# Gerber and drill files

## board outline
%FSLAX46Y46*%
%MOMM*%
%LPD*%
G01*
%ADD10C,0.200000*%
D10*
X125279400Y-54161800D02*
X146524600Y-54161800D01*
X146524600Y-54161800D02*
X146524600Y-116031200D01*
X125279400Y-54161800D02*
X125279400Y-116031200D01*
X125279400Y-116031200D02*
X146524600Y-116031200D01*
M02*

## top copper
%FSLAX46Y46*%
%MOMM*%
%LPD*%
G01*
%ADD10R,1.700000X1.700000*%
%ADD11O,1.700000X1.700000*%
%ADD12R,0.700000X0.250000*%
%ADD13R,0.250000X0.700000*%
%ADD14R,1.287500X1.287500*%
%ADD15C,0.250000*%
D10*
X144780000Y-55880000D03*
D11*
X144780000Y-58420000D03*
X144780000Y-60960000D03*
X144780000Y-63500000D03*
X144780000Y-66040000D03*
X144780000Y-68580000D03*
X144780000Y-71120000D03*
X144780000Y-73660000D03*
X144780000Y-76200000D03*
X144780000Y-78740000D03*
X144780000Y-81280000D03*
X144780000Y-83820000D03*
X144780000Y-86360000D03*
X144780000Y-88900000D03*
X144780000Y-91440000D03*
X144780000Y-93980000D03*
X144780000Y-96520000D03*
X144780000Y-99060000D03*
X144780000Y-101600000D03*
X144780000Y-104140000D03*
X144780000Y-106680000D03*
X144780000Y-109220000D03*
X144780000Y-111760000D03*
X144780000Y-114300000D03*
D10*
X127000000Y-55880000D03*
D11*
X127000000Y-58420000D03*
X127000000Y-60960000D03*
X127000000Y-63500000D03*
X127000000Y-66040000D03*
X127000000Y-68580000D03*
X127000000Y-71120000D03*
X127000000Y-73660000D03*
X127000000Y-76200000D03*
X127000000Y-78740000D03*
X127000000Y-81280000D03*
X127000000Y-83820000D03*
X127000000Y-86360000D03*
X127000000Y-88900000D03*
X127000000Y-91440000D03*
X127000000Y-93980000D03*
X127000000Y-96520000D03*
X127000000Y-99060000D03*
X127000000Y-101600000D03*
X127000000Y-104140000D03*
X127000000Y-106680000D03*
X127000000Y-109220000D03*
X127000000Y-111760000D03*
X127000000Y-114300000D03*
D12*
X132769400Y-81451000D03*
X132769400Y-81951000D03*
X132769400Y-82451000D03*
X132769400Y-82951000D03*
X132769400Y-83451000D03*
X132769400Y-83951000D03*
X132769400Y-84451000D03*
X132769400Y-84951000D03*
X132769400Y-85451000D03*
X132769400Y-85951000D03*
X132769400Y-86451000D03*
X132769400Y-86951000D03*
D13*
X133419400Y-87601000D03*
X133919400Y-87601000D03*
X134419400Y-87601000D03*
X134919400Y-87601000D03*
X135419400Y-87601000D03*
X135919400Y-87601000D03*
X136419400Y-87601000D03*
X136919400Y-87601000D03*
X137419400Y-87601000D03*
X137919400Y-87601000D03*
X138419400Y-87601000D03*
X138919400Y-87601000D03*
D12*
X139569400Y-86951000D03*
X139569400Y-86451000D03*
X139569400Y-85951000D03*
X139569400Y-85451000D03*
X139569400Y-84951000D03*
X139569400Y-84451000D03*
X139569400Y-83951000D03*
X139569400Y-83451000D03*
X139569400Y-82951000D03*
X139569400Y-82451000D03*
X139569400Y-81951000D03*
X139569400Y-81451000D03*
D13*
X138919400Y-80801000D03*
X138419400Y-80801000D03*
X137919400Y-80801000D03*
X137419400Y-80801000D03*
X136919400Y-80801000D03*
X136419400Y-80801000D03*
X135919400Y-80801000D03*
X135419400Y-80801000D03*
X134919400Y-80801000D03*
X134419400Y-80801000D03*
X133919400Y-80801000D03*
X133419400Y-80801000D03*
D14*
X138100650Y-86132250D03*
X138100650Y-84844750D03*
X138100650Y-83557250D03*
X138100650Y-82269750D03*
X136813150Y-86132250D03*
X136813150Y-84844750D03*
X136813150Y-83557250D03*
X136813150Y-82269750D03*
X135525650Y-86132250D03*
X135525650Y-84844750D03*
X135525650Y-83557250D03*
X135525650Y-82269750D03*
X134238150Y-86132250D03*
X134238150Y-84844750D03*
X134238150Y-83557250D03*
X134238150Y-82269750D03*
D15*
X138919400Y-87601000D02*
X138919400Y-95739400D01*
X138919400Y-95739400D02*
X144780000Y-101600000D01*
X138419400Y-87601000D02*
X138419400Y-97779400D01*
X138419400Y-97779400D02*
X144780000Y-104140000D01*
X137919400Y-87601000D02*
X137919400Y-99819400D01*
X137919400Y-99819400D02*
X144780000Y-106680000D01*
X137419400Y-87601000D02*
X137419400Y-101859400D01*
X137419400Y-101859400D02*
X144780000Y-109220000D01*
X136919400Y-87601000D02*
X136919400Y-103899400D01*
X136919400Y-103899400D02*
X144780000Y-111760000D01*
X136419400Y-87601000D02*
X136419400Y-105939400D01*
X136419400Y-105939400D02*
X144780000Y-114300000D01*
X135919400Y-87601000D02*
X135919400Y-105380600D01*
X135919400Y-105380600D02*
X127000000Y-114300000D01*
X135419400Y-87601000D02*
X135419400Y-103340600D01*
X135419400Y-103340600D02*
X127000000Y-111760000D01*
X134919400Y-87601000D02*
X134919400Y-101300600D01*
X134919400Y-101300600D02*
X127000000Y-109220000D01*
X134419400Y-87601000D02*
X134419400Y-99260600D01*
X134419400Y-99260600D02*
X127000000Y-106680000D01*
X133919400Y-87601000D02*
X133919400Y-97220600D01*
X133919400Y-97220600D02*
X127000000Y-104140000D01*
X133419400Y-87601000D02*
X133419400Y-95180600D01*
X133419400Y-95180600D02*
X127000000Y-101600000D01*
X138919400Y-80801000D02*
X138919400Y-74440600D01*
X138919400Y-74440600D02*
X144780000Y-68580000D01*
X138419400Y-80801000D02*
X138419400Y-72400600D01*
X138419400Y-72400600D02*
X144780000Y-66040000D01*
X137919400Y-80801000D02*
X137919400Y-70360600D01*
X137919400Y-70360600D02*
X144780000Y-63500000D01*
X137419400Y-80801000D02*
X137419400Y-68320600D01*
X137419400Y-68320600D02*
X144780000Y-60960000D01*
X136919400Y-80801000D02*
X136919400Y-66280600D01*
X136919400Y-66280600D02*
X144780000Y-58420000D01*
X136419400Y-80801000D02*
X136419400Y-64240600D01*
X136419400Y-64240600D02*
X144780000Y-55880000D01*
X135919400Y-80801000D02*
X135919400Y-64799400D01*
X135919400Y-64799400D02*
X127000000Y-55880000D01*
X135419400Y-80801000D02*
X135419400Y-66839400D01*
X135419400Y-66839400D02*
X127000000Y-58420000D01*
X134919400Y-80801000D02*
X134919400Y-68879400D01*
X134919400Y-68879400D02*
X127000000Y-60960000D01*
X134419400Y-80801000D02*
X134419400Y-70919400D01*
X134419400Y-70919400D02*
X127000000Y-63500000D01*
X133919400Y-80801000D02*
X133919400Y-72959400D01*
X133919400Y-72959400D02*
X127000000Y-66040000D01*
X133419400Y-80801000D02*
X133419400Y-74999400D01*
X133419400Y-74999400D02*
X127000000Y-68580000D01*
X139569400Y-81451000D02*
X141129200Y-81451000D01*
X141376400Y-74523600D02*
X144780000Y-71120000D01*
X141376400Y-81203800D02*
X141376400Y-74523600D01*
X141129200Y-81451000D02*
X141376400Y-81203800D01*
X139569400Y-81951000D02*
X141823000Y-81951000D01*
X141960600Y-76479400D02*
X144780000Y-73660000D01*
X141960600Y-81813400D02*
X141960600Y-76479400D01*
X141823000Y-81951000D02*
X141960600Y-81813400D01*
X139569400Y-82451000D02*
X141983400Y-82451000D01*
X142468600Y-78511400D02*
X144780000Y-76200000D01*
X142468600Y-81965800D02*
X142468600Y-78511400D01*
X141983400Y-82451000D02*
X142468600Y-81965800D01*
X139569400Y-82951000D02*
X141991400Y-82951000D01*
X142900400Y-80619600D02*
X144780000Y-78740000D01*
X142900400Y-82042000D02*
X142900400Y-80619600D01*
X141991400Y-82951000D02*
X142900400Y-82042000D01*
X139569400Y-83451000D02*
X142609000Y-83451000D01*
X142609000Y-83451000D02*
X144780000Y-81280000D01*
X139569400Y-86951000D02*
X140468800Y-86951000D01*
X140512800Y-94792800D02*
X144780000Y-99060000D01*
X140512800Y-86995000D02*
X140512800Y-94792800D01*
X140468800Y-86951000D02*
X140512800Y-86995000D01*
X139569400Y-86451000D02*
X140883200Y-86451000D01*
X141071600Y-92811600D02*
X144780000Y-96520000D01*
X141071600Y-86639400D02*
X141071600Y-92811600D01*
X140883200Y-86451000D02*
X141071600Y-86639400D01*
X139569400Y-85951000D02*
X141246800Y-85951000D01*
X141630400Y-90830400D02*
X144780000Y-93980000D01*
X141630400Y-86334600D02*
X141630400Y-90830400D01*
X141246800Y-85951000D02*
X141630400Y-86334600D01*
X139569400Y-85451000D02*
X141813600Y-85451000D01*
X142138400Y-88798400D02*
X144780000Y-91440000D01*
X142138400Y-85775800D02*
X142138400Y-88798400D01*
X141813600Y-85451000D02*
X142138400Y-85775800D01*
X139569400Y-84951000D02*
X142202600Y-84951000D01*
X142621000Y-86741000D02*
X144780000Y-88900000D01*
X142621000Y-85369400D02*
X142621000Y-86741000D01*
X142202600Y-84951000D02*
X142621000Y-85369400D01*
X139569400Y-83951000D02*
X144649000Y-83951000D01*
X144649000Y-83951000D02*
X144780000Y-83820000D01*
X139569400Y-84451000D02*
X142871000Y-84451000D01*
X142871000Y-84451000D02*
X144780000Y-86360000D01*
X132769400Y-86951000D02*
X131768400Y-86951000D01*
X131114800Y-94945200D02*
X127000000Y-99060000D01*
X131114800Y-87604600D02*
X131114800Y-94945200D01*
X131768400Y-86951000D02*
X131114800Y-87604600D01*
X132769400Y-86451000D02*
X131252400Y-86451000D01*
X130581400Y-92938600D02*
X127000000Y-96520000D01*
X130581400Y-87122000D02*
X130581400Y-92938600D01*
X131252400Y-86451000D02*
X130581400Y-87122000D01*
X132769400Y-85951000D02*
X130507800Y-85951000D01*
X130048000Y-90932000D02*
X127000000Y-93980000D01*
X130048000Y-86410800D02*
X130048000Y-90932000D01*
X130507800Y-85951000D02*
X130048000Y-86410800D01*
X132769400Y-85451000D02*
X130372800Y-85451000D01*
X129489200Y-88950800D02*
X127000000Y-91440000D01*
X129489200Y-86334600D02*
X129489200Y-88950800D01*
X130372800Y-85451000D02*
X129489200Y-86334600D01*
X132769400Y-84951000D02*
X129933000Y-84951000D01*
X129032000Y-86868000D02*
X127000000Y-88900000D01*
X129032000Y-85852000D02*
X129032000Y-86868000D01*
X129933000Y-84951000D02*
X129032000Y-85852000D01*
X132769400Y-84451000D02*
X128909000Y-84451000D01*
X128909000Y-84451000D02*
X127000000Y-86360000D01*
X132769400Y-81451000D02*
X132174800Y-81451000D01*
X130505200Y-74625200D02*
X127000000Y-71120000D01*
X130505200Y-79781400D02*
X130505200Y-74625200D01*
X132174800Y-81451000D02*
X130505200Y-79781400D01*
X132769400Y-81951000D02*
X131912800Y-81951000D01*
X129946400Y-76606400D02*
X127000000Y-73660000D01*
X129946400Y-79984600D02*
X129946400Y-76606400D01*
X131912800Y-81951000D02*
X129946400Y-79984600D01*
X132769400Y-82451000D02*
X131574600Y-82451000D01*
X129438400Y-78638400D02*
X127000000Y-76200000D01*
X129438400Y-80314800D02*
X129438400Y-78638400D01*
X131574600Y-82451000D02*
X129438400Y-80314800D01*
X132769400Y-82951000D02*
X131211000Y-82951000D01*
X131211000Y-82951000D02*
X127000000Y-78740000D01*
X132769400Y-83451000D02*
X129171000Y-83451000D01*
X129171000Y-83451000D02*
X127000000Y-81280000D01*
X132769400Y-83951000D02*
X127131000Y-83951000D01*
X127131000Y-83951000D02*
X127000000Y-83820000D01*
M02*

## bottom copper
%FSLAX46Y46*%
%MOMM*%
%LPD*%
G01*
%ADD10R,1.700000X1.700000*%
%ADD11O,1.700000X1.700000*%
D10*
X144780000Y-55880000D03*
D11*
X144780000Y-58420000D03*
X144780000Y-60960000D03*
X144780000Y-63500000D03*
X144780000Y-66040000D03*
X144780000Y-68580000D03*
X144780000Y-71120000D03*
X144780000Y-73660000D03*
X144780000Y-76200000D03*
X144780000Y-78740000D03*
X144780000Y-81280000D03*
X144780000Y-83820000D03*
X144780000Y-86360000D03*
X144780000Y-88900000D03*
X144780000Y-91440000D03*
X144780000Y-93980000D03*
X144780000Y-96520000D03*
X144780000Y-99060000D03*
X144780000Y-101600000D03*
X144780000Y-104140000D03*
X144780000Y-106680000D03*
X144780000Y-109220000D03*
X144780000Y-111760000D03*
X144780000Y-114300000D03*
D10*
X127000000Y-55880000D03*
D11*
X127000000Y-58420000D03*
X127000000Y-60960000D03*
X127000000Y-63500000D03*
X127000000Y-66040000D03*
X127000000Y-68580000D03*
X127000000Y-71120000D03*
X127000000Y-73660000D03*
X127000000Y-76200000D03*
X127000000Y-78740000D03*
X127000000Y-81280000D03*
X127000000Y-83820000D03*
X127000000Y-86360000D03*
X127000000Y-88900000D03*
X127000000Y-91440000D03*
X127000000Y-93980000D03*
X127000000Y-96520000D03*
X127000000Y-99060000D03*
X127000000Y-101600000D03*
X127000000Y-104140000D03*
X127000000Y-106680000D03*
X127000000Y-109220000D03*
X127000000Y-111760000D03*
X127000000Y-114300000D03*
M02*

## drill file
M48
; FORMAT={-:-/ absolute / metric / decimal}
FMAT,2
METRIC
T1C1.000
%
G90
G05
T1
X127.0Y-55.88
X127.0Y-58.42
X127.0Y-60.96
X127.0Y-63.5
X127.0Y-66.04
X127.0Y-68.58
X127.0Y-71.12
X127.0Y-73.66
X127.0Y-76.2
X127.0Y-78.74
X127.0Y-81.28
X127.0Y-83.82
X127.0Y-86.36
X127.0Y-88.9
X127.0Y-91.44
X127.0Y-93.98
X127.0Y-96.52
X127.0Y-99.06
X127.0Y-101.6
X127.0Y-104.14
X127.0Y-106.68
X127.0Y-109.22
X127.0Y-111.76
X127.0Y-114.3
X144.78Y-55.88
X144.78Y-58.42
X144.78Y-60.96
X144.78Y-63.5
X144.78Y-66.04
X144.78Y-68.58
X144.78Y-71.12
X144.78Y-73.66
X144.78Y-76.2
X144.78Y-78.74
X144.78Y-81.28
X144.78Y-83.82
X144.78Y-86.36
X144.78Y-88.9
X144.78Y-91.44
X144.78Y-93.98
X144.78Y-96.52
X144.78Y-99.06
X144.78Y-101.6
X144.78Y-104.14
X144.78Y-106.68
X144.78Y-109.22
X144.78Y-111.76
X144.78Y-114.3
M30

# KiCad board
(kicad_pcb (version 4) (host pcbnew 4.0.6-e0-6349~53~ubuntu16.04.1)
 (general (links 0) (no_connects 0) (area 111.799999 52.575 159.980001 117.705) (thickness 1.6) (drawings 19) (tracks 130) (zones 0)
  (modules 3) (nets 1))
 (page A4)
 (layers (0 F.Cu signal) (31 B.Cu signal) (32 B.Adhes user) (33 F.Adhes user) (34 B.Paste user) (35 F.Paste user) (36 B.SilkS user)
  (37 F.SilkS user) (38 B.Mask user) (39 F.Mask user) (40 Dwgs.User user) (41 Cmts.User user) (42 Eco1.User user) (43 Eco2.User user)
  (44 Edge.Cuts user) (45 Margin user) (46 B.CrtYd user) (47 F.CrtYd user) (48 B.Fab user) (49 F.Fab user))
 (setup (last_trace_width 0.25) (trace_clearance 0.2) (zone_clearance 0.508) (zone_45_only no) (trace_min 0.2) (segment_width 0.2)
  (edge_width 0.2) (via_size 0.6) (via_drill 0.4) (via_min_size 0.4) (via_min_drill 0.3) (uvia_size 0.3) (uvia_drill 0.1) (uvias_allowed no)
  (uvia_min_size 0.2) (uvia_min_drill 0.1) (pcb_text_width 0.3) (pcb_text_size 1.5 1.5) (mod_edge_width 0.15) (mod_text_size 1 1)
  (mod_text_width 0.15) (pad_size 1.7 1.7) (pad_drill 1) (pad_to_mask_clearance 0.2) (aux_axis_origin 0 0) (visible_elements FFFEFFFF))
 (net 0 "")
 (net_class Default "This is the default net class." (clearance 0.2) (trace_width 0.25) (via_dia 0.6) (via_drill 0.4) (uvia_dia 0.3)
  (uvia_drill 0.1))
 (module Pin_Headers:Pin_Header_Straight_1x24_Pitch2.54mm (layer F.Cu) (at 144.78 55.88)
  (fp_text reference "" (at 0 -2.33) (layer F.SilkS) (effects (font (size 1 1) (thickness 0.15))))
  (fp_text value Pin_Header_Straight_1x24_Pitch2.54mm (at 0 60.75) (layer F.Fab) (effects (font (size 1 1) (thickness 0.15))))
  (pad 1 thru_hole rect (at 0 0) (size 1.7 1.7) (drill 1) (layers *.Cu *.Mask))
  (pad 2 thru_hole oval (at 0 2.54) (size 1.7 1.7) (drill 1) (layers *.Cu *.Mask))
  (pad 3 thru_hole oval (at 0 5.08) (size 1.7 1.7) (drill 1) (layers *.Cu *.Mask))
  (pad 4 thru_hole oval (at 0 7.62) (size 1.7 1.7) (drill 1) (layers *.Cu *.Mask))
  (pad 5 thru_hole oval (at 0 10.16) (size 1.7 1.7) (drill 1) (layers *.Cu *.Mask))
  (pad 6 thru_hole oval (at 0 12.7) (size 1.7 1.7) (drill 1) (layers *.Cu *.Mask))
  (pad 7 thru_hole oval (at 0 15.24) (size 1.7 1.7) (drill 1) (layers *.Cu *.Mask))
  (pad 8 thru_hole oval (at 0 17.78) (size 1.7 1.7) (drill 1) (layers *.Cu *.Mask))
  (pad 9 thru_hole oval (at 0 20.32) (size 1.7 1.7) (drill 1) (layers *.Cu *.Mask))
  (pad 10 thru_hole oval (at 0 22.86) (size 1.7 1.7) (drill 1) (layers *.Cu *.Mask))
  (pad 11 thru_hole oval (at 0 25.4) (size 1.7 1.7) (drill 1) (layers *.Cu *.Mask))
  (pad 12 thru_hole oval (at 0 27.94) (size 1.7 1.7) (drill 1) (layers *.Cu *.Mask))
  (pad 13 thru_hole oval (at 0 30.48) (size 1.7 1.7) (drill 1) (layers *.Cu *.Mask))
  (pad 14 thru_hole oval (at 0 33.02) (size 1.7 1.7) (drill 1) (layers *.Cu *.Mask))
  (pad 15 thru_hole oval (at 0 35.56) (size 1.7 1.7) (drill 1) (layers *.Cu *.Mask))
  (pad 16 thru_hole oval (at 0 38.1) (size 1.7 1.7) (drill 1) (layers *.Cu *.Mask))
  (pad 17 thru_hole oval (at 0 40.64) (size 1.7 1.7) (drill 1) (layers *.Cu *.Mask))
  (pad 18 thru_hole oval (at 0 43.18) (size 1.7 1.7) (drill 1) (layers *.Cu *.Mask))
  (pad 19 thru_hole oval (at 0 45.72) (size 1.7 1.7) (drill 1) (layers *.Cu *.Mask))
  (pad 20 thru_hole oval (at 0 48.26) (size 1.7 1.7) (drill 1) (layers *.Cu *.Mask))
  (pad 21 thru_hole oval (at 0 50.8) (size 1.7 1.7) (drill 1) (layers *.Cu *.Mask))
  (pad 22 thru_hole oval (at 0 53.34) (size 1.7 1.7) (drill 1) (layers *.Cu *.Mask))
  (pad 23 thru_hole oval (at 0 55.88) (size 1.7 1.7) (drill 1) (layers *.Cu *.Mask))
  (pad 24 thru_hole oval (at 0 58.42) (size 1.7 1.7) (drill 1) (layers *.Cu *.Mask)))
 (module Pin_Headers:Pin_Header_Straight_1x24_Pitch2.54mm (layer F.Cu) (at 127 55.88)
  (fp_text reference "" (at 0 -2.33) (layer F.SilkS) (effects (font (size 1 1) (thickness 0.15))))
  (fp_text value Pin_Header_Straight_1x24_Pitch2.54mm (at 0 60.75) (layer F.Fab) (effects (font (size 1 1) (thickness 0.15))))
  (pad 1 thru_hole rect (at 0 0) (size 1.7 1.7) (drill 1) (layers *.Cu *.Mask))
  (pad 2 thru_hole oval (at 0 2.54) (size 1.7 1.7) (drill 1) (layers *.Cu *.Mask))
  (pad 3 thru_hole oval (at 0 5.08) (size 1.7 1.7) (drill 1) (layers *.Cu *.Mask))
  (pad 4 thru_hole oval (at 0 7.62) (size 1.7 1.7) (drill 1) (layers *.Cu *.Mask))
  (pad 5 thru_hole oval (at 0 10.16) (size 1.7 1.7) (drill 1) (layers *.Cu *.Mask))
  (pad 6 thru_hole oval (at 0 12.7) (size 1.7 1.7) (drill 1) (layers *.Cu *.Mask))
  (pad 7 thru_hole oval (at 0 15.24) (size 1.7 1.7) (drill 1) (layers *.Cu *.Mask))
  (pad 8 thru_hole oval (at 0 17.78) (size 1.7 1.7) (drill 1) (layers *.Cu *.Mask))
  (pad 9 thru_hole oval (at 0 20.32) (size 1.7 1.7) (drill 1) (layers *.Cu *.Mask))
  (pad 10 thru_hole oval (at 0 22.86) (size 1.7 1.7) (drill 1) (layers *.Cu *.Mask))
  (pad 11 thru_hole oval (at 0 25.4) (size 1.7 1.7) (drill 1) (layers *.Cu *.Mask))
  (pad 12 thru_hole oval (at 0 27.94) (size 1.7 1.7) (drill 1) (layers *.Cu *.Mask))
  (pad 13 thru_hole oval (at 0 30.48) (size 1.7 1.7) (drill 1) (layers *.Cu *.Mask))
  (pad 14 thru_hole oval (at 0 33.02) (size 1.7 1.7) (drill 1) (layers *.Cu *.Mask))
  (pad 15 thru_hole oval (at 0 35.56) (size 1.7 1.7) (drill 1) (layers *.Cu *.Mask))
  (pad 16 thru_hole oval (at 0 38.1) (size 1.7 1.7) (drill 1) (layers *.Cu *.Mask))
  (pad 17 thru_hole oval (at 0 40.64) (size 1.7 1.7) (drill 1) (layers *.Cu *.Mask))
  (pad 18 thru_hole oval (at 0 43.18) (size 1.7 1.7) (drill 1) (layers *.Cu *.Mask))
  (pad 19 thru_hole oval (at 0 45.72) (size 1.7 1.7) (drill 1) (layers *.Cu *.Mask))
  (pad 20 thru_hole oval (at 0 48.26) (size 1.7 1.7) (drill 1) (layers *.Cu *.Mask))
  (pad 21 thru_hole oval (at 0 50.8) (size 1.7 1.7) (drill 1) (layers *.Cu *.Mask))
  (pad 22 thru_hole oval (at 0 53.34) (size 1.7 1.7) (drill 1) (layers *.Cu *.Mask))
  (pad 23 thru_hole oval (at 0 55.88) (size 1.7 1.7) (drill 1) (layers *.Cu *.Mask))
  (pad 24 thru_hole oval (at 0 58.42) (size 1.7 1.7) (drill 1) (layers *.Cu *.Mask)))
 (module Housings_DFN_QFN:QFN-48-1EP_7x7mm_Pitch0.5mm (layer F.Cu) (at 136.1694 84.201)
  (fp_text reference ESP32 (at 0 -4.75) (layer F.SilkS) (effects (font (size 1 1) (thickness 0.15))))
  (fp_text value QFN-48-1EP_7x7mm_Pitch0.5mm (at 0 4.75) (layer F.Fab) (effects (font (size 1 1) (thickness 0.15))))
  (pad 1 smd rect (at -3.4 -2.75) (size 0.7 0.25) (layers F.Cu F.Paste F.Mask))
  (pad 2 smd rect (at -3.4 -2.25) (size 0.7 0.25) (layers F.Cu F.Paste F.Mask))
  (pad 3 smd rect (at -3.4 -1.75) (size 0.7 0.25) (layers F.Cu F.Paste F.Mask))
  (pad 4 smd rect (at -3.4 -1.25) (size 0.7 0.25) (layers F.Cu F.Paste F.Mask))
  (pad 5 smd rect (at -3.4 -0.75) (size 0.7 0.25) (layers F.Cu F.Paste F.Mask))
  (pad 6 smd rect (at -3.4 -0.25) (size 0.7 0.25) (layers F.Cu F.Paste F.Mask))
  (pad 7 smd rect (at -3.4 0.25) (size 0.7 0.25) (layers F.Cu F.Paste F.Mask))
  (pad 8 smd rect (at -3.4 0.75) (size 0.7 0.25) (layers F.Cu F.Paste F.Mask))
  (pad 9 smd rect (at -3.4 1.25) (size 0.7 0.25) (layers F.Cu F.Paste F.Mask))
  (pad 10 smd rect (at -3.4 1.75) (size 0.7 0.25) (layers F.Cu F.Paste F.Mask))
  (pad 11 smd rect (at -3.4 2.25) (size 0.7 0.25) (layers F.Cu F.Paste F.Mask))
  (pad 12 smd rect (at -3.4 2.75) (size 0.7 0.25) (layers F.Cu F.Paste F.Mask))
  (pad 13 smd rect (at -2.75 3.4 90) (size 0.7 0.25) (layers F.Cu F.Paste F.Mask))
  (pad 14 smd rect (at -2.25 3.4 90) (size 0.7 0.25) (layers F.Cu F.Paste F.Mask))
  (pad 15 smd rect (at -1.75 3.4 90) (size 0.7 0.25) (layers F.Cu F.Paste F.Mask))
  (pad 16 smd rect (at -1.25 3.4 90) (size 0.7 0.25) (layers F.Cu F.Paste F.Mask))
  (pad 17 smd rect (at -0.75 3.4 90) (size 0.7 0.25) (layers F.Cu F.Paste F.Mask))
  (pad 18 smd rect (at -0.25 3.4 90) (size 0.7 0.25) (layers F.Cu F.Paste F.Mask))
  (pad 19 smd rect (at 0.25 3.4 90) (size 0.7 0.25) (layers F.Cu F.Paste F.Mask))
  (pad 20 smd rect (at 0.75 3.4 90) (size 0.7 0.25) (layers F.Cu F.Paste F.Mask))
  (pad 21 smd rect (at 1.25 3.4 90) (size 0.7 0.25) (layers F.Cu F.Paste F.Mask))
  (pad 22 smd rect (at 1.75 3.4 90) (size 0.7 0.25) (layers F.Cu F.Paste F.Mask))
  (pad 23 smd rect (at 2.25 3.4 90) (size 0.7 0.25) (layers F.Cu F.Paste F.Mask))
  (pad 24 smd rect (at 2.75 3.4 90) (size 0.7 0.25) (layers F.Cu F.Paste F.Mask))
  (pad 25 smd rect (at 3.4 2.75) (size 0.7 0.25) (layers F.Cu F.Paste F.Mask))
  (pad 26 smd rect (at 3.4 2.25) (size 0.7 0.25) (layers F.Cu F.Paste F.Mask))
  (pad 27 smd rect (at 3.4 1.75) (size 0.7 0.25) (layers F.Cu F.Paste F.Mask))
  (pad 28 smd rect (at 3.4 1.25) (size 0.7 0.25) (layers F.Cu F.Paste F.Mask))
  (pad 29 smd rect (at 3.4 0.75) (size 0.7 0.25) (layers F.Cu F.Paste F.Mask))
  (pad 30 smd rect (at 3.4 0.25) (size 0.7 0.25) (layers F.Cu F.Paste F.Mask))
  (pad 31 smd rect (at 3.4 -0.25) (size 0.7 0.25) (layers F.Cu F.Paste F.Mask))
  (pad 32 smd rect (at 3.4 -0.75) (size 0.7 0.25) (layers F.Cu F.Paste F.Mask))
  (pad 33 smd rect (at 3.4 -1.25) (size 0.7 0.25) (layers F.Cu F.Paste F.Mask))
  (pad 34 smd rect (at 3.4 -1.75) (size 0.7 0.25) (layers F.Cu F.Paste F.Mask))
  (pad 35 smd rect (at 3.4 -2.25) (size 0.7 0.25) (layers F.Cu F.Paste F.Mask))
  (pad 36 smd rect (at 3.4 -2.75) (size 0.7 0.25) (layers F.Cu F.Paste F.Mask))
  (pad 37 smd rect (at 2.75 -3.4 90) (size 0.7 0.25) (layers F.Cu F.Paste F.Mask))
  (pad 38 smd rect (at 2.25 -3.4 90) (size 0.7 0.25) (layers F.Cu F.Paste F.Mask))
  (pad 39 smd rect (at 1.75 -3.4 90) (size 0.7 0.25) (layers F.Cu F.Paste F.Mask))
  (pad 40 smd rect (at 1.25 -3.4 90) (size 0.7 0.25) (layers F.Cu F.Paste F.Mask))
  (pad 41 smd rect (at 0.75 -3.4 90) (size 0.7 0.25) (layers F.Cu F.Paste F.Mask))
  (pad 42 smd rect (at 0.25 -3.4 90) (size 0.7 0.25) (layers F.Cu F.Paste F.Mask))
  (pad 43 smd rect (at -0.25 -3.4 90) (size 0.7 0.25) (layers F.Cu F.Paste F.Mask))
  (pad 44 smd rect (at -0.75 -3.4 90) (size 0.7 0.25) (layers F.Cu F.Paste F.Mask))
  (pad 45 smd rect (at -1.25 -3.4 90) (size 0.7 0.25) (layers F.Cu F.Paste F.Mask))
  (pad 46 smd rect (at -1.75 -3.4 90) (size 0.7 0.25) (layers F.Cu F.Paste F.Mask))
  (pad 47 smd rect (at -2.25 -3.4 90) (size 0.7 0.25) (layers F.Cu F.Paste F.Mask))
  (pad 48 smd rect (at -2.75 -3.4 90) (size 0.7 0.25) (layers F.Cu F.Paste F.Mask))
  (pad 49 smd rect (at 1.93125 1.93125) (size 1.2875 1.2875) (layers F.Cu F.Paste F.Mask) (solder_paste_margin_ratio -0.2))
  (pad 49 smd rect (at 1.93125 0.64375) (size 1.2875 1.2875) (layers F.Cu F.Paste F.Mask) (solder_paste_margin_ratio -0.2))
  (pad 49 smd rect (at 1.93125 -0.64375) (size 1.2875 1.2875) (layers F.Cu F.Paste F.Mask) (solder_paste_margin_ratio -0.2))
  (pad 49 smd rect (at 1.93125 -1.93125) (size 1.2875 1.2875) (layers F.Cu F.Paste F.Mask) (solder_paste_margin_ratio -0.2))
  (pad 49 smd rect (at 0.64375 1.93125) (size 1.2875 1.2875) (layers F.Cu F.Paste F.Mask) (solder_paste_margin_ratio -0.2))
  (pad 49 smd rect (at 0.64375 0.64375) (size 1.2875 1.2875) (layers F.Cu F.Paste F.Mask) (solder_paste_margin_ratio -0.2))
  (pad 49 smd rect (at 0.64375 -0.64375) (size 1.2875 1.2875) (layers F.Cu F.Paste F.Mask) (solder_paste_margin_ratio -0.2))
  (pad 49 smd rect (at 0.64375 -1.93125) (size 1.2875 1.2875) (layers F.Cu F.Paste F.Mask) (solder_paste_margin_ratio -0.2))
  (pad 49 smd rect (at -0.64375 1.93125) (size 1.2875 1.2875) (layers F.Cu F.Paste F.Mask) (solder_paste_margin_ratio -0.2))
  (pad 49 smd rect (at -0.64375 0.64375) (size 1.2875 1.2875) (layers F.Cu F.Paste F.Mask) (solder_paste_margin_ratio -0.2))
  (pad 49 smd rect (at -0.64375 -0.64375) (size 1.2875 1.2875) (layers F.Cu F.Paste F.Mask) (solder_paste_margin_ratio -0.2))
  (pad 49 smd rect (at -0.64375 -1.93125) (size 1.2875 1.2875) (layers F.Cu F.Paste F.Mask) (solder_paste_margin_ratio -0.2))
  (pad 49 smd rect (at -1.93125 1.93125) (size 1.2875 1.2875) (layers F.Cu F.Paste F.Mask) (solder_paste_margin_ratio -0.2))
  (pad 49 smd rect (at -1.93125 0.64375) (size 1.2875 1.2875) (layers F.Cu F.Paste F.Mask) (solder_paste_margin_ratio -0.2))
  (pad 49 smd rect (at -1.93125 -0.64375) (size 1.2875 1.2875) (layers F.Cu F.Paste F.Mask) (solder_paste_margin_ratio -0.2))
  (pad 49 smd rect (at -1.93125 -1.93125) (size 1.2875 1.2875) (layers F.Cu F.Paste F.Mask) (solder_paste_margin_ratio -0.2)))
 (gr_line (start 125.2794 54.1618) (end 146.5246 54.1618) (angle 90) (layer Edge.Cuts) (width 0.2))
 (gr_line (start 146.5246 54.1618) (end 146.5246 116.0312) (angle 90) (layer Edge.Cuts) (width 0.2))
 (gr_line (start 125.2794 54.1618) (end 125.2794 116.0312) (angle 90) (layer Edge.Cuts) (width 0.2))
 (gr_line (start 125.2794 116.0312) (end 146.5246 116.0312) (angle 90) (layer Edge.Cuts) (width 0.2))
 (segment (start 138.9194 87.601) (end 138.9194 95.7394) (width 0.25) (layer F.Cu) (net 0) (status 400000))
 (segment (start 138.9194 95.7394) (end 144.78 101.6) (width 0.25) (layer F.Cu) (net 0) (status 800000))
 (segment (start 138.4194 87.601) (end 138.4194 97.7794) (width 0.25) (layer F.Cu) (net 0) (status 400000))
 (segment (start 138.4194 97.7794) (end 144.78 104.14) (width 0.25) (layer F.Cu) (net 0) (status 800000))
 (segment (start 137.9194 87.601) (end 137.9194 99.8194) (width 0.25) (layer F.Cu) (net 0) (status 400000))
 (segment (start 137.9194 99.8194) (end 144.78 106.68) (width 0.25) (layer F.Cu) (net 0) (status 800000))
 (segment (start 137.4194 87.601) (end 137.4194 101.8594) (width 0.25) (layer F.Cu) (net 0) (status 400000))
 (segment (start 137.4194 101.8594) (end 144.78 109.22) (width 0.25) (layer F.Cu) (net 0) (status 800000))
 (segment (start 136.9194 87.601) (end 136.9194 103.8994) (width 0.25) (layer F.Cu) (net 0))
 (segment (start 136.9194 103.8994) (end 144.78 111.76) (width 0.25) (layer F.Cu) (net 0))
 (segment (start 136.4194 87.601) (end 136.4194 105.9394) (width 0.25) (layer F.Cu) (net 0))
 (segment (start 136.4194 105.9394) (end 144.78 114.3) (width 0.25) (layer F.Cu) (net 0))
 (segment (start 135.9194 87.601) (end 135.9194 105.3806) (width 0.25) (layer F.Cu) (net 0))
 (segment (start 135.9194 105.3806) (end 127 114.3) (width 0.25) (layer F.Cu) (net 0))
 (segment (start 135.4194 87.601) (end 135.4194 103.3406) (width 0.25) (layer F.Cu) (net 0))
 (segment (start 135.4194 103.3406) (end 127 111.76) (width 0.25) (layer F.Cu) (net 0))
 (segment (start 134.9194 87.601) (end 134.9194 101.3006) (width 0.25) (layer F.Cu) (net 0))
 (segment (start 134.9194 101.3006) (end 127 109.22) (width 0.25) (layer F.Cu) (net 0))
 (segment (start 134.4194 87.601) (end 134.4194 99.2606) (width 0.25) (layer F.Cu) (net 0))
 (segment (start 134.4194 99.2606) (end 127 106.68) (width 0.25) (layer F.Cu) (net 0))
 (segment (start 133.9194 87.601) (end 133.9194 97.2206) (width 0.25) (layer F.Cu) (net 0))
 (segment (start 133.9194 97.2206) (end 127 104.14) (width 0.25) (layer F.Cu) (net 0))
 (segment (start 133.4194 87.601) (end 133.4194 95.1806) (width 0.25) (layer F.Cu) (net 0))
 (segment (start 133.4194 95.1806) (end 127 101.6) (width 0.25) (layer F.Cu) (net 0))
 (segment (start 138.9194 80.801) (end 138.9194 74.4406) (width 0.25) (layer F.Cu) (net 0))
 (segment (start 138.9194 74.4406) (end 144.78 68.58) (width 0.25) (layer F.Cu) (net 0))
 (segment (start 138.4194 80.801) (end 138.4194 72.4006) (width 0.25) (layer F.Cu) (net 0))
 (segment (start 138.4194 72.4006) (end 144.78 66.04) (width 0.25) (layer F.Cu) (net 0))
 (segment (start 137.9194 80.801) (end 137.9194 70.3606) (width 0.25) (layer F.Cu) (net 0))
 (segment (start 137.9194 70.3606) (end 144.78 63.5) (width 0.25) (layer F.Cu) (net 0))
 (segment (start 137.4194 80.801) (end 137.4194 68.3206) (width 0.25) (layer F.Cu) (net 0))
 (segment (start 137.4194 68.3206) (end 144.78 60.96) (width 0.25) (layer F.Cu) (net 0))
 (segment (start 136.9194 80.801) (end 136.9194 66.2806) (width 0.25) (layer F.Cu) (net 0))
 (segment (start 136.9194 66.2806) (end 144.78 58.42) (width 0.25) (layer F.Cu) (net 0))
 (segment (start 136.4194 80.801) (end 136.4194 64.2406) (width 0.25) (layer F.Cu) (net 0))
 (segment (start 136.4194 64.2406) (end 144.78 55.88) (width 0.25) (layer F.Cu) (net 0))
 (segment (start 135.9194 80.801) (end 135.9194 64.7994) (width 0.25) (layer F.Cu) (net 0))
 (segment (start 135.9194 64.7994) (end 127 55.88) (width 0.25) (layer F.Cu) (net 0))
 (segment (start 135.4194 80.801) (end 135.4194 66.8394) (width 0.25) (layer F.Cu) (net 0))
 (segment (start 135.4194 66.8394) (end 127 58.42) (width 0.25) (layer F.Cu) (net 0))
 (segment (start 134.9194 80.801) (end 134.9194 68.8794) (width 0.25) (layer F.Cu) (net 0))
 (segment (start 134.9194 68.8794) (end 127 60.96) (width 0.25) (layer F.Cu) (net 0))
 (segment (start 134.4194 80.801) (end 134.4194 70.9194) (width 0.25) (layer F.Cu) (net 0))
 (segment (start 134.4194 70.9194) (end 127 63.5) (width 0.25) (layer F.Cu) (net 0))
 (segment (start 133.9194 80.801) (end 133.9194 72.9594) (width 0.25) (layer F.Cu) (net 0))
 (segment (start 133.9194 72.9594) (end 127 66.04) (width 0.25) (layer F.Cu) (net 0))
 (segment (start 133.4194 80.801) (end 133.4194 74.9994) (width 0.25) (layer F.Cu) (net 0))
 (segment (start 133.4194 74.9994) (end 127 68.58) (width 0.25) (layer F.Cu) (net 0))
 (segment (start 139.5694 81.451) (end 141.1292 81.451) (width 0.25) (layer F.Cu) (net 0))
 (segment (start 141.3764 74.5236) (end 144.78 71.12) (width 0.25) (layer F.Cu) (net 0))
 (segment (start 141.3764 81.2038) (end 141.3764 74.5236) (width 0.25) (layer F.Cu) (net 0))
 (segment (start 141.1292 81.451) (end 141.3764 81.2038) (width 0.25) (layer F.Cu) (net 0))
 (segment (start 139.5694 81.951) (end 141.823 81.951) (width 0.25) (layer F.Cu) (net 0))
 (segment (start 141.9606 76.4794) (end 144.78 73.66) (width 0.25) (layer F.Cu) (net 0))
 (segment (start 141.9606 81.8134) (end 141.9606 76.4794) (width 0.25) (layer F.Cu) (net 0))
 (segment (start 141.823 81.951) (end 141.9606 81.8134) (width 0.25) (layer F.Cu) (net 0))
 (segment (start 139.5694 82.451) (end 141.9834 82.451) (width 0.25) (layer F.Cu) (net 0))
 (segment (start 142.4686 78.5114) (end 144.78 76.2) (width 0.25) (layer F.Cu) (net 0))
 (segment (start 142.4686 81.9658) (end 142.4686 78.5114) (width 0.25) (layer F.Cu) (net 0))
 (segment (start 141.9834 82.451) (end 142.4686 81.9658) (width 0.25) (layer F.Cu) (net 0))
 (segment (start 139.5694 82.951) (end 141.9914 82.951) (width 0.25) (layer F.Cu) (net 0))
 (segment (start 142.9004 80.6196) (end 144.78 78.74) (width 0.25) (layer F.Cu) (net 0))
 (segment (start 142.9004 82.042) (end 142.9004 80.6196) (width 0.25) (layer F.Cu) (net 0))
 (segment (start 141.9914 82.951) (end 142.9004 82.042) (width 0.25) (layer F.Cu) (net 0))
 (segment (start 139.5694 83.451) (end 142.609 83.451) (width 0.25) (layer F.Cu) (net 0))
 (segment (start 142.609 83.451) (end 144.78 81.28) (width 0.25) (layer F.Cu) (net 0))
 (segment (start 139.5694 86.951) (end 140.4688 86.951) (width 0.25) (layer F.Cu) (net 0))
 (segment (start 140.5128 94.7928) (end 144.78 99.06) (width 0.25) (layer F.Cu) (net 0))
 (segment (start 140.5128 86.995) (end 140.5128 94.7928) (width 0.25) (layer F.Cu) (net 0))
 (segment (start 140.4688 86.951) (end 140.5128 86.995) (width 0.25) (layer F.Cu) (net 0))
 (segment (start 139.5694 86.451) (end 140.8832 86.451) (width 0.25) (layer F.Cu) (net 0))
 (segment (start 141.0716 92.8116) (end 144.78 96.52) (width 0.25) (layer F.Cu) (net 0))
 (segment (start 141.0716 86.6394) (end 141.0716 92.8116) (width 0.25) (layer F.Cu) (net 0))
 (segment (start 140.8832 86.451) (end 141.0716 86.6394) (width 0.25) (layer F.Cu) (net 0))
 (segment (start 139.5694 85.951) (end 141.2468 85.951) (width 0.25) (layer F.Cu) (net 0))
 (segment (start 141.6304 90.8304) (end 144.78 93.98) (width 0.25) (layer F.Cu) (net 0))
 (segment (start 141.6304 86.3346) (end 141.6304 90.8304) (width 0.25) (layer F.Cu) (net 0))
 (segment (start 141.2468 85.951) (end 141.6304 86.3346) (width 0.25) (layer F.Cu) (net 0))
 (segment (start 139.5694 85.451) (end 141.8136 85.451) (width 0.25) (layer F.Cu) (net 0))
 (segment (start 142.1384 88.7984) (end 144.78 91.44) (width 0.25) (layer F.Cu) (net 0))
 (segment (start 142.1384 85.7758) (end 142.1384 88.7984) (width 0.25) (layer F.Cu) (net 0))
 (segment (start 141.8136 85.451) (end 142.1384 85.7758) (width 0.25) (layer F.Cu) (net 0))
 (segment (start 139.5694 84.951) (end 142.2026 84.951) (width 0.25) (layer F.Cu) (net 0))
 (segment (start 142.621 86.741) (end 144.78 88.9) (width 0.25) (layer F.Cu) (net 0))
 (segment (start 142.621 85.3694) (end 142.621 86.741) (width 0.25) (layer F.Cu) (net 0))
 (segment (start 142.2026 84.951) (end 142.621 85.3694) (width 0.25) (layer F.Cu) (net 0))
 (segment (start 139.5694 83.951) (end 144.649 83.951) (width 0.25) (layer F.Cu) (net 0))
 (segment (start 144.649 83.951) (end 144.78 83.82) (width 0.25) (layer F.Cu) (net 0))
 (segment (start 139.5694 84.451) (end 142.871 84.451) (width 0.25) (layer F.Cu) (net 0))
 (segment (start 142.871 84.451) (end 144.78 86.36) (width 0.25) (layer F.Cu) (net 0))
 (segment (start 132.7694 86.951) (end 131.7684 86.951) (width 0.25) (layer F.Cu) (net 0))
 (segment (start 131.1148 94.9452) (end 127 99.06) (width 0.25) (layer F.Cu) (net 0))
 (segment (start 131.1148 87.6046) (end 131.1148 94.9452) (width 0.25) (layer F.Cu) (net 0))
 (segment (start 131.7684 86.951) (end 131.1148 87.6046) (width 0.25) (layer F.Cu) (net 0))
 (segment (start 132.7694 86.451) (end 131.2524 86.451) (width 0.25) (layer F.Cu) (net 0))
 (segment (start 130.5814 92.9386) (end 127 96.52) (width 0.25) (layer F.Cu) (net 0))
 (segment (start 130.5814 87.122) (end 130.5814 92.9386) (width 0.25) (layer F.Cu) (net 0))
 (segment (start 131.2524 86.451) (end 130.5814 87.122) (width 0.25) (layer F.Cu) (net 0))
 (segment (start 132.7694 85.951) (end 130.5078 85.951) (width 0.25) (layer F.Cu) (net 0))
 (segment (start 130.048 90.932) (end 127 93.98) (width 0.25) (layer F.Cu) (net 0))
 (segment (start 130.048 86.4108) (end 130.048 90.932) (width 0.25) (layer F.Cu) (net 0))
 (segment (start 130.5078 85.951) (end 130.048 86.4108) (width 0.25) (layer F.Cu) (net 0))
 (segment (start 132.7694 85.451) (end 130.3728 85.451) (width 0.25) (layer F.Cu) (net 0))
 (segment (start 129.4892 88.9508) (end 127 91.44) (width 0.25) (layer F.Cu) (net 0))
 (segment (start 129.4892 86.3346) (end 129.4892 88.9508) (width 0.25) (layer F.Cu) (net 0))
 (segment (start 130.3728 85.451) (end 129.4892 86.3346) (width 0.25) (layer F.Cu) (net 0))
 (segment (start 132.7694 84.951) (end 129.933 84.951) (width 0.25) (layer F.Cu) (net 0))
 (segment (start 129.032 86.868) (end 127 88.9) (width 0.25) (layer F.Cu) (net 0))
 (segment (start 129.032 85.852) (end 129.032 86.868) (width 0.25) (layer F.Cu) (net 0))
 (segment (start 129.933 84.951) (end 129.032 85.852) (width 0.25) (layer F.Cu) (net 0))
 (segment (start 132.7694 84.451) (end 128.909 84.451) (width 0.25) (layer F.Cu) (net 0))
 (segment (start 128.909 84.451) (end 127 86.36) (width 0.25) (layer F.Cu) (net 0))
 (segment (start 132.7694 81.451) (end 132.1748 81.451) (width 0.25) (layer F.Cu) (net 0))
 (segment (start 130.5052 74.6252) (end 127 71.12) (width 0.25) (layer F.Cu) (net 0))
 (segment (start 130.5052 79.7814) (end 130.5052 74.6252) (width 0.25) (layer F.Cu) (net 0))
 (segment (start 132.1748 81.451) (end 130.5052 79.7814) (width 0.25) (layer F.Cu) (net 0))
 (segment (start 132.7694 81.951) (end 131.9128 81.951) (width 0.25) (layer F.Cu) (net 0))
 (segment (start 129.9464 76.6064) (end 127 73.66) (width 0.25) (layer F.Cu) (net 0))
 (segment (start 129.9464 79.9846) (end 129.9464 76.6064) (width 0.25) (layer F.Cu) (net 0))
 (segment (start 131.9128 81.951) (end 129.9464 79.9846) (width 0.25) (layer F.Cu) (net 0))
 (segment (start 132.7694 82.451) (end 131.5746 82.451) (width 0.25) (layer F.Cu) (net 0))
 (segment (start 129.4384 78.6384) (end 127 76.2) (width 0.25) (layer F.Cu) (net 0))
 (segment (start 129.4384 80.3148) (end 129.4384 78.6384) (width 0.25) (layer F.Cu) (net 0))
 (segment (start 131.5746 82.451) (end 129.4384 80.3148) (width 0.25) (layer F.Cu) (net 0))
 (segment (start 132.7694 82.951) (end 131.211 82.951) (width 0.25) (layer F.Cu) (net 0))
 (segment (start 131.211 82.951) (end 127 78.74) (width 0.25) (layer F.Cu) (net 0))
 (segment (start 132.7694 83.451) (end 129.171 83.451) (width 0.25) (layer F.Cu) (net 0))
 (segment (start 129.171 83.451) (end 127 81.28) (width 0.25) (layer F.Cu) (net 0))
 (segment (start 132.7694 83.951) (end 127.131 83.951) (width 0.25) (layer F.Cu) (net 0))
 (segment (start 127.131 83.951) (end 127 83.82) (width 0.25) (layer F.Cu) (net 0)))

